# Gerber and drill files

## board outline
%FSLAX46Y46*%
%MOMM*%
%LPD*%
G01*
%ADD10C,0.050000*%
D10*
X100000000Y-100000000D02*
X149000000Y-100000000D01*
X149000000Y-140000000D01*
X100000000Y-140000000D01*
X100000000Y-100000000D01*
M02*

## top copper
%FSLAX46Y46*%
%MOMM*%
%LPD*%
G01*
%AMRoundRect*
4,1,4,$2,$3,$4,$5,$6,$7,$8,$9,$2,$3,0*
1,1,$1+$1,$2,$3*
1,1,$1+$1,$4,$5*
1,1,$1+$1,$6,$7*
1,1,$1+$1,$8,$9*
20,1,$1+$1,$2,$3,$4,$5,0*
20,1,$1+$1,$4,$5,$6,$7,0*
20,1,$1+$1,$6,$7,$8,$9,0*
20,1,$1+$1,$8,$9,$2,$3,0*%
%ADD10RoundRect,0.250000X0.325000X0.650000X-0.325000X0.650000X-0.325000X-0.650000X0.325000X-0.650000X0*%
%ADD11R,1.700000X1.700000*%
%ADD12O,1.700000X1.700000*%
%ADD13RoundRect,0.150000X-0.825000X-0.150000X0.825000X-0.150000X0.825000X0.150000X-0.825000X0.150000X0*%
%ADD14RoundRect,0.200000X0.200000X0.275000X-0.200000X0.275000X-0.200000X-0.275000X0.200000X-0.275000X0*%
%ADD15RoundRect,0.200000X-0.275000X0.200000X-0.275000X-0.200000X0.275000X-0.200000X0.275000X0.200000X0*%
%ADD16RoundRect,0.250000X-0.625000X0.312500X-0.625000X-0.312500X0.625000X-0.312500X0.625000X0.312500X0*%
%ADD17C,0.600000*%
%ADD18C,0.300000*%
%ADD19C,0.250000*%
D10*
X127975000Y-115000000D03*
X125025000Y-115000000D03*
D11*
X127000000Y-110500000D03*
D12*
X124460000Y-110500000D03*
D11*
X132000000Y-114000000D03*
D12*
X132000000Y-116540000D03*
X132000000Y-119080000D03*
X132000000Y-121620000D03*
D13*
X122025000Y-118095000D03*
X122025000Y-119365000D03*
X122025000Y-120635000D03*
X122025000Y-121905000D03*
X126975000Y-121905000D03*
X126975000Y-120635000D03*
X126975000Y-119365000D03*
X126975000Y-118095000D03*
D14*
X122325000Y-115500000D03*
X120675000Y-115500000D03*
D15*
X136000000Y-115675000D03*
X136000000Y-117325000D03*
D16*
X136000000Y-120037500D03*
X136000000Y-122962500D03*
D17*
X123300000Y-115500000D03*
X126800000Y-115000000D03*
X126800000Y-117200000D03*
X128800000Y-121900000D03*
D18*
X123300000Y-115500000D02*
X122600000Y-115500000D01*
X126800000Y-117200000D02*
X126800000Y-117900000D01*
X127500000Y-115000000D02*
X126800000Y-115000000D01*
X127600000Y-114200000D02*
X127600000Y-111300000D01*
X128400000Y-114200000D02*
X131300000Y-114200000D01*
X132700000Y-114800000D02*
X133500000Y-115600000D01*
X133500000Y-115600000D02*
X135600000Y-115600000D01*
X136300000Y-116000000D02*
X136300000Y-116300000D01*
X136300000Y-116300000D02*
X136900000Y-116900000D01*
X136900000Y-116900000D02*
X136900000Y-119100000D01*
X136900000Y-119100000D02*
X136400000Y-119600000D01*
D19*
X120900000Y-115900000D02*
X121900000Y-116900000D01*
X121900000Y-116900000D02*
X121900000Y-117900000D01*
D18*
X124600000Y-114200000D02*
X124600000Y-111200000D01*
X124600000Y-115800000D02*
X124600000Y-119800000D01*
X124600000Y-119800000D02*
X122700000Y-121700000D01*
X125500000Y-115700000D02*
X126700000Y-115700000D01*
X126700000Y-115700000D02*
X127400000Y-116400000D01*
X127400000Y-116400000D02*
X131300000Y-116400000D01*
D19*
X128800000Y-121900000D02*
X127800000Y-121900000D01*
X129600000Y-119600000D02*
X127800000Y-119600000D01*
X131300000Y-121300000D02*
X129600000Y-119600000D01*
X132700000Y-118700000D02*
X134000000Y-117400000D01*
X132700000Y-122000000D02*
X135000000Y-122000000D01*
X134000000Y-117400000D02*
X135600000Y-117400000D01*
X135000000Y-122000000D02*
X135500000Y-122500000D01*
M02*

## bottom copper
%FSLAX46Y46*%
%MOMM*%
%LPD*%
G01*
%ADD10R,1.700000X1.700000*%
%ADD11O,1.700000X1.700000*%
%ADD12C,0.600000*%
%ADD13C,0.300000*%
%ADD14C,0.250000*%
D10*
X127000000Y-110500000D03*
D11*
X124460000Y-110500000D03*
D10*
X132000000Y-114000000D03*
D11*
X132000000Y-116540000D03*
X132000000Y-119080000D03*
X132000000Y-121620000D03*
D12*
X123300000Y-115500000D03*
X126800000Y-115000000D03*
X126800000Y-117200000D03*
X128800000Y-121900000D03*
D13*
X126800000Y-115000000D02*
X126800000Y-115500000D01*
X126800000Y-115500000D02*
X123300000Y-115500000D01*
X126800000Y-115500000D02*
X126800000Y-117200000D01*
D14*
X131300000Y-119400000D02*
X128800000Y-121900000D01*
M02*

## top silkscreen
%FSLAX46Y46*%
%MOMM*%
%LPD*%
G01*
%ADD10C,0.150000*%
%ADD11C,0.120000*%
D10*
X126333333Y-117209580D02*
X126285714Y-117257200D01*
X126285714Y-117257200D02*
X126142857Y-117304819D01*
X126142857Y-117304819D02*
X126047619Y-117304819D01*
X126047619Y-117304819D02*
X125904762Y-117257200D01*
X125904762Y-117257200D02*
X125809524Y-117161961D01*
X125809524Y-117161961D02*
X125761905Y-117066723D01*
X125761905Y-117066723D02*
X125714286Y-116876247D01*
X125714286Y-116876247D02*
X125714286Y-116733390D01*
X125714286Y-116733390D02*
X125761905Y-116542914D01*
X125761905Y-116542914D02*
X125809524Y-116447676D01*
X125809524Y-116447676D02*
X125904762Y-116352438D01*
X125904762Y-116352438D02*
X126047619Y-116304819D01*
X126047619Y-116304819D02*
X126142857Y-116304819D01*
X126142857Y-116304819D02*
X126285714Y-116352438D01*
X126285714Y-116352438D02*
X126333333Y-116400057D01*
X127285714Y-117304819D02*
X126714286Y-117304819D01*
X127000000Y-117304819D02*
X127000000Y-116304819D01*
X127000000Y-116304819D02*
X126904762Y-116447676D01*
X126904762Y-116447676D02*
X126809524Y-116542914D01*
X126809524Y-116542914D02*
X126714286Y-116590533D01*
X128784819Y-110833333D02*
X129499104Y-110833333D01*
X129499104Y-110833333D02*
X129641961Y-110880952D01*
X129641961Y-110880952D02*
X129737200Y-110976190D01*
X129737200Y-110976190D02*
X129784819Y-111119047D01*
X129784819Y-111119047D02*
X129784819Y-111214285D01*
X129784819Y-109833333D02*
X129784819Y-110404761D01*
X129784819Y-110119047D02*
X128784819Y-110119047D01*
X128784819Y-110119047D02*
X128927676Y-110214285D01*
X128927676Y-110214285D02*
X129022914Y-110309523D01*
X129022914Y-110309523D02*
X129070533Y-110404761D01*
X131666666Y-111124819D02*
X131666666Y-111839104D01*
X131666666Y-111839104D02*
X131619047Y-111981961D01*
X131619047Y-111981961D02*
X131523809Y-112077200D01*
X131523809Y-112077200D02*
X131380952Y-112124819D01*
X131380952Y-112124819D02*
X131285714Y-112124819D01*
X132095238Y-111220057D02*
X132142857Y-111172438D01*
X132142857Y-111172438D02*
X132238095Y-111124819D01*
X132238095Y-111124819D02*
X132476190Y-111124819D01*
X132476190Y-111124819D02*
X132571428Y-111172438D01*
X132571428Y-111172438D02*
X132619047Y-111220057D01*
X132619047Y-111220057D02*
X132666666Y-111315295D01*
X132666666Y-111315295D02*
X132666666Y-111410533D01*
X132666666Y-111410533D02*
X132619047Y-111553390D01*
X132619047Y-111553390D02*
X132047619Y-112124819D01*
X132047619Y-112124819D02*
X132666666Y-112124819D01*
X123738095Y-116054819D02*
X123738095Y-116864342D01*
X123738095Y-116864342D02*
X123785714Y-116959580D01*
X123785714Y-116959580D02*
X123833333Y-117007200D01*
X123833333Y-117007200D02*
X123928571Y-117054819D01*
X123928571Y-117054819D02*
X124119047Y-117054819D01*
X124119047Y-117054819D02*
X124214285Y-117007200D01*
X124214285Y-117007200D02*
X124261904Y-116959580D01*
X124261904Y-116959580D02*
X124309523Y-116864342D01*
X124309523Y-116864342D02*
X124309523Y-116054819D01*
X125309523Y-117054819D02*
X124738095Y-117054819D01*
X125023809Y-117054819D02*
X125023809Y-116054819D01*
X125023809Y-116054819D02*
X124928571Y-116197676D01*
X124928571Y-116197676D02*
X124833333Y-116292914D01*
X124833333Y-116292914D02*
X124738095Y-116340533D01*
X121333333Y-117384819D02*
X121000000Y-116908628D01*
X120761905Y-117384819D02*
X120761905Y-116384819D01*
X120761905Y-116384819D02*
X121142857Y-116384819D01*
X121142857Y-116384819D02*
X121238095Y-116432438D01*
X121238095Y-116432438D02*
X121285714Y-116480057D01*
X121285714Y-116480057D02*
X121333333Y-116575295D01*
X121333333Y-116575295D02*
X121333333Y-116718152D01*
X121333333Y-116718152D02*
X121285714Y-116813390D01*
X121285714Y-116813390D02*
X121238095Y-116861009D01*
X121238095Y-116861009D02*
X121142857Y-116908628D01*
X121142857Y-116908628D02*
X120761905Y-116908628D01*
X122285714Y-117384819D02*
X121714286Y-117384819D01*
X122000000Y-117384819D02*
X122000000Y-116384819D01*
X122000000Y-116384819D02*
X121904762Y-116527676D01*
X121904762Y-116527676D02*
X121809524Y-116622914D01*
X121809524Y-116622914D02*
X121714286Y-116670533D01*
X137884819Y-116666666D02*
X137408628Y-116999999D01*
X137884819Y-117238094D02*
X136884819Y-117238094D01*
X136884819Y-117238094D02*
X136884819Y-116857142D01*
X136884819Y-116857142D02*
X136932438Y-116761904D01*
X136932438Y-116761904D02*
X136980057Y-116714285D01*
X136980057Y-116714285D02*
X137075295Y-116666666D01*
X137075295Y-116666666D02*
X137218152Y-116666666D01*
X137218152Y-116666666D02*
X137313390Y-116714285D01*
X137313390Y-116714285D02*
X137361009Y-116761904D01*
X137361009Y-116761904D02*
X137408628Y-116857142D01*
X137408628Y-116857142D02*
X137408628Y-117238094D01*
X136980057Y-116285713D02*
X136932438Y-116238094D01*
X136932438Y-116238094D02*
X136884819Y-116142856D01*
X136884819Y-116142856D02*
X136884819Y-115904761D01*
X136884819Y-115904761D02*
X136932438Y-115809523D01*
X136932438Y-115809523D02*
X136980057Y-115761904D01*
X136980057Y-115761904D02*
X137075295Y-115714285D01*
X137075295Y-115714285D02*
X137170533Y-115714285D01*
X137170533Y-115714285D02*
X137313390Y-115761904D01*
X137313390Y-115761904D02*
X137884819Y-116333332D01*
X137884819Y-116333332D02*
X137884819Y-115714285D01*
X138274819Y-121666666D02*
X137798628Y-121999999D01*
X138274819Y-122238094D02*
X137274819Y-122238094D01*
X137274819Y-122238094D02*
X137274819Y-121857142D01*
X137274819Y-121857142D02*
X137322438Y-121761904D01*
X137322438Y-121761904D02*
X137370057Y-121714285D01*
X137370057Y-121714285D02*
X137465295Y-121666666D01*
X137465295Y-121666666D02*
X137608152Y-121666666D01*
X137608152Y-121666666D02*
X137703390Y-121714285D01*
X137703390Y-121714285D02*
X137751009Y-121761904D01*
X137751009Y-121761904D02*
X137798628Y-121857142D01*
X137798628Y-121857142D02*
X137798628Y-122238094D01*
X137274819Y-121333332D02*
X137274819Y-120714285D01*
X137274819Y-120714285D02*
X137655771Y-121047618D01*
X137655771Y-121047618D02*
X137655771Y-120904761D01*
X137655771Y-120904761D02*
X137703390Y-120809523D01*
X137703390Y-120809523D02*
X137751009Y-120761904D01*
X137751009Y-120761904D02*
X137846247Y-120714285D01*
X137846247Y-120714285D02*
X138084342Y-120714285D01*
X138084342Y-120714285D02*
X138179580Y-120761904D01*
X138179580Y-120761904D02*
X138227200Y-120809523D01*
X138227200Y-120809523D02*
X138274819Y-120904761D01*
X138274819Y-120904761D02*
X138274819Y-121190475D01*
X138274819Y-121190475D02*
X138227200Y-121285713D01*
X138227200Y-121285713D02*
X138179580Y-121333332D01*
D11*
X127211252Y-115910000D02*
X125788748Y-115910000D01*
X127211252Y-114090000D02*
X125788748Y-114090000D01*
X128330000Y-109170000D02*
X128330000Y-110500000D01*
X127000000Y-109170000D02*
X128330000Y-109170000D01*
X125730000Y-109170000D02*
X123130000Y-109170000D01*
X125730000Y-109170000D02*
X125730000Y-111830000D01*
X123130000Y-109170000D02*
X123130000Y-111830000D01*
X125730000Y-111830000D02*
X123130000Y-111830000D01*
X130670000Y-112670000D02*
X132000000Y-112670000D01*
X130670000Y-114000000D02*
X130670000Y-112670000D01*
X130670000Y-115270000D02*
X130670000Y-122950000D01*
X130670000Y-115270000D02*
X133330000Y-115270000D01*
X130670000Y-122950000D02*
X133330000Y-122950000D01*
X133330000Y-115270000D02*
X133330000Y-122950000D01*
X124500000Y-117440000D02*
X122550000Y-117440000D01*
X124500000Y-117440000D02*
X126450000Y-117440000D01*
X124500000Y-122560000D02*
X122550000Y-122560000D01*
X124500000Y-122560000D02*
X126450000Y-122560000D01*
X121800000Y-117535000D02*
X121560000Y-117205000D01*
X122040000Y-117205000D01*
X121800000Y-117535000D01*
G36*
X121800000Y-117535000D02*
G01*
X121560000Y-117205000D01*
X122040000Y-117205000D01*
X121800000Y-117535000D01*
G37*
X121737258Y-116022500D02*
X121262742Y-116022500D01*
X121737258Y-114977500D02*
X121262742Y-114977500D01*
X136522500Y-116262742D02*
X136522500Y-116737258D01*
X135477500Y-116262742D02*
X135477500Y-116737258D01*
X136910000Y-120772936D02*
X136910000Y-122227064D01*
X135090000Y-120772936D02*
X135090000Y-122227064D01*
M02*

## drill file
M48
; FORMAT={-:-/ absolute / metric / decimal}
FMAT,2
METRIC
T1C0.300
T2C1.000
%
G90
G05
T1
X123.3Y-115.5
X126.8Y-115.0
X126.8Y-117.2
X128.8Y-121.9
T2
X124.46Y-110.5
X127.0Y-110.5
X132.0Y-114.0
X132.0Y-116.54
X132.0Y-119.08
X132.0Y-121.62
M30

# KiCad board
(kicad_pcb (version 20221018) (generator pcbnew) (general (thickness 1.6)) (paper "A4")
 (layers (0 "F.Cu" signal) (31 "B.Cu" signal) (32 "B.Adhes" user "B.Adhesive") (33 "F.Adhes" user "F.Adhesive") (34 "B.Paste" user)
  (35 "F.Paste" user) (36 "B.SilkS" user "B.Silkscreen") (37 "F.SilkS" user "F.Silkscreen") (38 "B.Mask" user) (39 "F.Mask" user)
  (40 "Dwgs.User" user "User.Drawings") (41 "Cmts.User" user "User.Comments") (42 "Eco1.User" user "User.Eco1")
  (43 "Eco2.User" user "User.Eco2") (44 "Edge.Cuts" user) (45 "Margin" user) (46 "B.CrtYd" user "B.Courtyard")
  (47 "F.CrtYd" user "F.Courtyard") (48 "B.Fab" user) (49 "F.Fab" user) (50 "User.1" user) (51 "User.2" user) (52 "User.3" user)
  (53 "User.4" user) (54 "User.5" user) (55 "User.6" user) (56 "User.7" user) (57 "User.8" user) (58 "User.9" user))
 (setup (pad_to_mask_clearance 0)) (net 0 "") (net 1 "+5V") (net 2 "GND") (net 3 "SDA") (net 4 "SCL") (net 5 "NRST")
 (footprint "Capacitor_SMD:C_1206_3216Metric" (layer "F.Cu") (at 126.5 115 180)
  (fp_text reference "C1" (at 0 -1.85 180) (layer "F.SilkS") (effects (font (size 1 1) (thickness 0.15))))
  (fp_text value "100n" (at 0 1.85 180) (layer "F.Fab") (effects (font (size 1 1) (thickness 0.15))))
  (fp_line (start -0.711252 -0.91) (end 0.711252 -0.91) (stroke (width 0.12) (type solid)) (layer "F.SilkS"))
  (fp_line (start -0.711252 0.91) (end 0.711252 0.91) (stroke (width 0.12) (type solid)) (layer "F.SilkS"))
  (pad "1" smd roundrect (at -1.475 0 180) (size 1.15 1.8) (layers "F.Cu" "F.Paste" "F.Mask") (roundrect_rratio 0.217391) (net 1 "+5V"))
  (pad "2" smd roundrect (at 1.475 0 180) (size 1.15 1.8) (layers "F.Cu" "F.Paste" "F.Mask") (roundrect_rratio 0.217391) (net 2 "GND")))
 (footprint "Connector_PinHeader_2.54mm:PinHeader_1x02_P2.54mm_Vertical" (layer "F.Cu") (at 127 110.5 -90)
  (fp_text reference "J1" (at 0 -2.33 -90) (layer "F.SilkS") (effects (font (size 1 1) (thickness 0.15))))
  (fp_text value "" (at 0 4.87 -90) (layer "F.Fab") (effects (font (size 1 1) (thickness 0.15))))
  (fp_line (start -1.33 -1.33) (end 0 -1.33) (stroke (width 0.12) (type solid)) (layer "F.SilkS"))
  (fp_line (start -1.33 0) (end -1.33 -1.33) (stroke (width 0.12) (type solid)) (layer "F.SilkS"))
  (fp_line (start -1.33 1.27) (end -1.33 3.87) (stroke (width 0.12) (type solid)) (layer "F.SilkS"))
  (fp_line (start -1.33 1.27) (end 1.33 1.27) (stroke (width 0.12) (type solid)) (layer "F.SilkS"))
  (fp_line (start -1.33 3.87) (end 1.33 3.87) (stroke (width 0.12) (type solid)) (layer "F.SilkS"))
  (fp_line (start 1.33 1.27) (end 1.33 3.87) (stroke (width 0.12) (type solid)) (layer "F.SilkS"))
  (pad "1" thru_hole rect (at 0 0 270) (size 1.7 1.7) (drill 1) (layers "*.Cu" "*.Mask") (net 1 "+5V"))
  (pad "2" thru_hole oval (at 0 2.54 270) (size 1.7 1.7) (drill 1) (layers "*.Cu" "*.Mask") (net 2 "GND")))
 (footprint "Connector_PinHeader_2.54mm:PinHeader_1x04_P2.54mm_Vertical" (layer "F.Cu") (at 132 114)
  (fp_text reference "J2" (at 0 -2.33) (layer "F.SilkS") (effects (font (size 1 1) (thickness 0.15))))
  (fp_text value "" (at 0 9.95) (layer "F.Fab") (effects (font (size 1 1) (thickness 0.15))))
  (fp_line (start -1.33 -1.33) (end 0 -1.33) (stroke (width 0.12) (type solid)) (layer "F.SilkS"))
  (fp_line (start -1.33 0) (end -1.33 -1.33) (stroke (width 0.12) (type solid)) (layer "F.SilkS"))
  (fp_line (start -1.33 1.27) (end -1.33 8.95) (stroke (width 0.12) (type solid)) (layer "F.SilkS"))
  (fp_line (start -1.33 1.27) (end 1.33 1.27) (stroke (width 0.12) (type solid)) (layer "F.SilkS"))
  (fp_line (start -1.33 8.95) (end 1.33 8.95) (stroke (width 0.12) (type solid)) (layer "F.SilkS"))
  (fp_line (start 1.33 1.27) (end 1.33 8.95) (stroke (width 0.12) (type solid)) (layer "F.SilkS"))
  (pad "1" thru_hole rect (at 0 0) (size 1.7 1.7) (drill 1) (layers "*.Cu" "*.Mask") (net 1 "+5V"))
  (pad "2" thru_hole oval (at 0 2.54) (size 1.7 1.7) (drill 1) (layers "*.Cu" "*.Mask") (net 2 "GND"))
  (pad "3" thru_hole oval (at 0 5.08) (size 1.7 1.7) (drill 1) (layers "*.Cu" "*.Mask") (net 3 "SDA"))
  (pad "4" thru_hole oval (at 0 7.62) (size 1.7 1.7) (drill 1) (layers "*.Cu" "*.Mask") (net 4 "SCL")))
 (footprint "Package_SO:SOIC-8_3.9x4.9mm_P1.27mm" (layer "F.Cu") (at 124.5 120)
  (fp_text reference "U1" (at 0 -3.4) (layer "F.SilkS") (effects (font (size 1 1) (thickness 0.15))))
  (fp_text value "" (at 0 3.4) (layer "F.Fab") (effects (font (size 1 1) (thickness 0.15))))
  (fp_line (start 0 -2.56) (end -1.95 -2.56) (stroke (width 0.12) (type solid)) (layer "F.SilkS"))
  (fp_line (start 0 -2.56) (end 1.95 -2.56) (stroke (width 0.12) (type solid)) (layer "F.SilkS"))
  (fp_line (start 0 2.56) (end -1.95 2.56) (stroke (width 0.12) (type solid)) (layer "F.SilkS"))
  (fp_line (start 0 2.56) (end 1.95 2.56) (stroke (width 0.12) (type solid)) (layer "F.SilkS"))
  (fp_poly
   (pts (xy -2.7 -2.465) (xy -2.94 -2.795) (xy -2.46 -2.795) (xy -2.7 -2.465)) (stroke (width 0.12) (type solid)) (fill solid)
   (layer "F.SilkS"))
  (pad "1" smd roundrect (at -2.475 -1.905) (size 1.95 0.6) (layers "F.Cu" "F.Paste" "F.Mask") (roundrect_rratio 0.25) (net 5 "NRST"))
  (pad "2" smd roundrect (at -2.475 -0.635) (size 1.95 0.6) (layers "F.Cu" "F.Paste" "F.Mask") (roundrect_rratio 0.25))
  (pad "3" smd roundrect (at -2.475 0.635) (size 1.95 0.6) (layers "F.Cu" "F.Paste" "F.Mask") (roundrect_rratio 0.25))
  (pad "4" smd roundrect (at -2.475 1.905) (size 1.95 0.6) (layers "F.Cu" "F.Paste" "F.Mask") (roundrect_rratio 0.25) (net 2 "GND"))
  (pad "5" smd roundrect (at 2.475 1.905) (size 1.95 0.6) (layers "F.Cu" "F.Paste" "F.Mask") (roundrect_rratio 0.25) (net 3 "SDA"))
  (pad "6" smd roundrect (at 2.475 0.635) (size 1.95 0.6) (layers "F.Cu" "F.Paste" "F.Mask") (roundrect_rratio 0.25))
  (pad "7" smd roundrect (at 2.475 -0.635) (size 1.95 0.6) (layers "F.Cu" "F.Paste" "F.Mask") (roundrect_rratio 0.25) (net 4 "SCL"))
  (pad "8" smd roundrect (at 2.475 -1.905) (size 1.95 0.6) (layers "F.Cu" "F.Paste" "F.Mask") (roundrect_rratio 0.25) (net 1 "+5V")))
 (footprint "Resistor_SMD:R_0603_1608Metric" (layer "F.Cu") (at 121.5 115.5 180)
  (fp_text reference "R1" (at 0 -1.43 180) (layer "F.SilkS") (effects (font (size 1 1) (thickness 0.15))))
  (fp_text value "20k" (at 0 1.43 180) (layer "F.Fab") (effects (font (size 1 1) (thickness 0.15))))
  (fp_line (start -0.237258 -0.5225) (end 0.237258 -0.5225) (stroke (width 0.12) (type solid)) (layer "F.SilkS"))
  (fp_line (start -0.237258 0.5225) (end 0.237258 0.5225) (stroke (width 0.12) (type solid)) (layer "F.SilkS"))
  (pad "1" smd roundrect (at -0.825 0 180) (size 0.8 0.95) (layers "F.Cu" "F.Paste" "F.Mask") (roundrect_rratio 0.25) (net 1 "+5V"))
  (pad "2" smd roundrect (at 0.825 0 180) (size 0.8 0.95) (layers "F.Cu" "F.Paste" "F.Mask") (roundrect_rratio 0.25) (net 5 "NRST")))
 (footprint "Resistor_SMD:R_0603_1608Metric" (layer "F.Cu") (at 136 116.5 -90)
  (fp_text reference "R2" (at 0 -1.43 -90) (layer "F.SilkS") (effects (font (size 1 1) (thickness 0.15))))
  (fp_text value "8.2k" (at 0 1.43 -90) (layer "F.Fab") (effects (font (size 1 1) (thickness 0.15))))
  (fp_line (start -0.237258 -0.5225) (end 0.237258 -0.5225) (stroke (width 0.12) (type solid)) (layer "F.SilkS"))
  (fp_line (start -0.237258 0.5225) (end 0.237258 0.5225) (stroke (width 0.12) (type solid)) (layer "F.SilkS"))
  (pad "1" smd roundrect (at -0.825 0 270) (size 0.8 0.95) (layers "F.Cu" "F.Paste" "F.Mask") (roundrect_rratio 0.25) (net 1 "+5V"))
  (pad "2" smd roundrect (at 0.825 0 270) (size 0.8 0.95) (layers "F.Cu" "F.Paste" "F.Mask") (roundrect_rratio 0.25) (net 3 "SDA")))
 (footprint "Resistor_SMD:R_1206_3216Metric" (layer "F.Cu") (at 136 121.5 -90)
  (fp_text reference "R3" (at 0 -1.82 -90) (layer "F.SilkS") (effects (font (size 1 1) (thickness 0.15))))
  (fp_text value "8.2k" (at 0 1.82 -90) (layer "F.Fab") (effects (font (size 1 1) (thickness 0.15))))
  (fp_line (start -0.727064 -0.91) (end 0.727064 -0.91) (stroke (width 0.12) (type solid)) (layer "F.SilkS"))
  (fp_line (start -0.727064 0.91) (end 0.727064 0.91) (stroke (width 0.12) (type solid)) (layer "F.SilkS"))
  (pad "1" smd roundrect (at -1.4625 0 270) (size 1.125 1.75) (layers "F.Cu" "F.Paste" "F.Mask") (roundrect_rratio 0.222222) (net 1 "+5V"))
  (pad "2" smd roundrect (at 1.4625 0 270) (size 1.125 1.75) (layers "F.Cu" "F.Paste" "F.Mask") (roundrect_rratio 0.222222) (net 4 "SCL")))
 (gr_rect (start 100 100) (end 149 140) (stroke (width 0.05) (type default)) (fill none) (layer "Edge.Cuts"))
 (segment (start 123.3 115.5) (end 122.6 115.5) (width 0.3) (layer "F.Cu") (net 1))
 (segment (start 126.8 117.2) (end 126.8 117.9) (width 0.3) (layer "F.Cu") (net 1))
 (segment (start 127.5 115) (end 126.8 115) (width 0.3) (layer "F.Cu") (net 1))
 (segment (start 127.6 114.2) (end 127.6 111.3) (width 0.3) (layer "F.Cu") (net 1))
 (segment (start 128.4 114.2) (end 131.3 114.2) (width 0.3) (layer "F.Cu") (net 1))
 (segment (start 132.7 114.8) (end 133.5 115.6) (width 0.3) (layer "F.Cu") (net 1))
 (segment (start 133.5 115.6) (end 135.6 115.6) (width 0.3) (layer "F.Cu") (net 1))
 (segment (start 136.3 116) (end 136.3 116.3) (width 0.3) (layer "F.Cu") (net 1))
 (segment (start 136.3 116.3) (end 136.9 116.9) (width 0.3) (layer "F.Cu") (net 1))
 (segment (start 136.9 116.9) (end 136.9 119.1) (width 0.3) (layer "F.Cu") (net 1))
 (segment (start 136.9 119.1) (end 136.4 119.6) (width 0.3) (layer "F.Cu") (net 1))
 (via (at 123.3 115.5) (size 0.6) (drill 0.3) (layers "F.Cu" "B.Cu") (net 1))
 (via (at 126.8 115) (size 0.6) (drill 0.3) (layers "F.Cu" "B.Cu") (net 1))
 (via (at 126.8 117.2) (size 0.6) (drill 0.3) (layers "F.Cu" "B.Cu") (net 1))
 (segment (start 120.9 115.9) (end 121.9 116.9) (width 0.25) (layer "F.Cu") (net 5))
 (segment (start 121.9 116.9) (end 121.9 117.9) (width 0.25) (layer "F.Cu") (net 5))
 (segment (start 124.6 114.2) (end 124.6 111.2) (width 0.3) (layer "F.Cu") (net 2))
 (segment (start 124.6 115.8) (end 124.6 119.8) (width 0.3) (layer "F.Cu") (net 2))
 (segment (start 124.6 119.8) (end 122.7 121.7) (width 0.3) (layer "F.Cu") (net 2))
 (segment (start 125.5 115.7) (end 126.7 115.7) (width 0.3) (layer "F.Cu") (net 2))
 (segment (start 126.7 115.7) (end 127.4 116.4) (width 0.3) (layer "F.Cu") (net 2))
 (segment (start 126.8 115) (end 126.8 115.5) (width 0.3) (layer "B.Cu") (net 1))
 (segment (start 126.8 115.5) (end 123.3 115.5) (width 0.3) (layer "B.Cu") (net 1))
 (segment (start 126.8 115.5) (end 126.8 117.2) (width 0.3) (layer "B.Cu") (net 1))
 (segment (start 127.4 116.4) (end 131.3 116.4) (width 0.3) (layer "F.Cu") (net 2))
 (segment (start 128.8 121.9) (end 127.8 121.9) (width 0.25) (layer "F.Cu") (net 3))
 (segment (start 129.6 119.6) (end 127.8 119.6) (width 0.25) (layer "F.Cu") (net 4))
 (segment (start 131.3 121.3) (end 129.6 119.6) (width 0.25) (layer "F.Cu") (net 4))
 (segment (start 132.7 118.7) (end 134 117.4) (width 0.25) (layer "F.Cu") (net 3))
 (segment (start 132.7 122) (end 135 122) (width 0.25) (layer "F.Cu") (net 4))
 (segment (start 134 117.4) (end 135.6 117.4) (width 0.25) (layer "F.Cu") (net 3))
 (segment (start 135 122) (end 135.5 122.5) (width 0.25) (layer "F.Cu") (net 4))
 (via (at 128.8 121.9) (size 0.6) (drill 0.3) (layers "F.Cu" "B.Cu") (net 3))
 (segment (start 131.3 119.4) (end 128.8 121.9) (width 0.25) (layer "B.Cu") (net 3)))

